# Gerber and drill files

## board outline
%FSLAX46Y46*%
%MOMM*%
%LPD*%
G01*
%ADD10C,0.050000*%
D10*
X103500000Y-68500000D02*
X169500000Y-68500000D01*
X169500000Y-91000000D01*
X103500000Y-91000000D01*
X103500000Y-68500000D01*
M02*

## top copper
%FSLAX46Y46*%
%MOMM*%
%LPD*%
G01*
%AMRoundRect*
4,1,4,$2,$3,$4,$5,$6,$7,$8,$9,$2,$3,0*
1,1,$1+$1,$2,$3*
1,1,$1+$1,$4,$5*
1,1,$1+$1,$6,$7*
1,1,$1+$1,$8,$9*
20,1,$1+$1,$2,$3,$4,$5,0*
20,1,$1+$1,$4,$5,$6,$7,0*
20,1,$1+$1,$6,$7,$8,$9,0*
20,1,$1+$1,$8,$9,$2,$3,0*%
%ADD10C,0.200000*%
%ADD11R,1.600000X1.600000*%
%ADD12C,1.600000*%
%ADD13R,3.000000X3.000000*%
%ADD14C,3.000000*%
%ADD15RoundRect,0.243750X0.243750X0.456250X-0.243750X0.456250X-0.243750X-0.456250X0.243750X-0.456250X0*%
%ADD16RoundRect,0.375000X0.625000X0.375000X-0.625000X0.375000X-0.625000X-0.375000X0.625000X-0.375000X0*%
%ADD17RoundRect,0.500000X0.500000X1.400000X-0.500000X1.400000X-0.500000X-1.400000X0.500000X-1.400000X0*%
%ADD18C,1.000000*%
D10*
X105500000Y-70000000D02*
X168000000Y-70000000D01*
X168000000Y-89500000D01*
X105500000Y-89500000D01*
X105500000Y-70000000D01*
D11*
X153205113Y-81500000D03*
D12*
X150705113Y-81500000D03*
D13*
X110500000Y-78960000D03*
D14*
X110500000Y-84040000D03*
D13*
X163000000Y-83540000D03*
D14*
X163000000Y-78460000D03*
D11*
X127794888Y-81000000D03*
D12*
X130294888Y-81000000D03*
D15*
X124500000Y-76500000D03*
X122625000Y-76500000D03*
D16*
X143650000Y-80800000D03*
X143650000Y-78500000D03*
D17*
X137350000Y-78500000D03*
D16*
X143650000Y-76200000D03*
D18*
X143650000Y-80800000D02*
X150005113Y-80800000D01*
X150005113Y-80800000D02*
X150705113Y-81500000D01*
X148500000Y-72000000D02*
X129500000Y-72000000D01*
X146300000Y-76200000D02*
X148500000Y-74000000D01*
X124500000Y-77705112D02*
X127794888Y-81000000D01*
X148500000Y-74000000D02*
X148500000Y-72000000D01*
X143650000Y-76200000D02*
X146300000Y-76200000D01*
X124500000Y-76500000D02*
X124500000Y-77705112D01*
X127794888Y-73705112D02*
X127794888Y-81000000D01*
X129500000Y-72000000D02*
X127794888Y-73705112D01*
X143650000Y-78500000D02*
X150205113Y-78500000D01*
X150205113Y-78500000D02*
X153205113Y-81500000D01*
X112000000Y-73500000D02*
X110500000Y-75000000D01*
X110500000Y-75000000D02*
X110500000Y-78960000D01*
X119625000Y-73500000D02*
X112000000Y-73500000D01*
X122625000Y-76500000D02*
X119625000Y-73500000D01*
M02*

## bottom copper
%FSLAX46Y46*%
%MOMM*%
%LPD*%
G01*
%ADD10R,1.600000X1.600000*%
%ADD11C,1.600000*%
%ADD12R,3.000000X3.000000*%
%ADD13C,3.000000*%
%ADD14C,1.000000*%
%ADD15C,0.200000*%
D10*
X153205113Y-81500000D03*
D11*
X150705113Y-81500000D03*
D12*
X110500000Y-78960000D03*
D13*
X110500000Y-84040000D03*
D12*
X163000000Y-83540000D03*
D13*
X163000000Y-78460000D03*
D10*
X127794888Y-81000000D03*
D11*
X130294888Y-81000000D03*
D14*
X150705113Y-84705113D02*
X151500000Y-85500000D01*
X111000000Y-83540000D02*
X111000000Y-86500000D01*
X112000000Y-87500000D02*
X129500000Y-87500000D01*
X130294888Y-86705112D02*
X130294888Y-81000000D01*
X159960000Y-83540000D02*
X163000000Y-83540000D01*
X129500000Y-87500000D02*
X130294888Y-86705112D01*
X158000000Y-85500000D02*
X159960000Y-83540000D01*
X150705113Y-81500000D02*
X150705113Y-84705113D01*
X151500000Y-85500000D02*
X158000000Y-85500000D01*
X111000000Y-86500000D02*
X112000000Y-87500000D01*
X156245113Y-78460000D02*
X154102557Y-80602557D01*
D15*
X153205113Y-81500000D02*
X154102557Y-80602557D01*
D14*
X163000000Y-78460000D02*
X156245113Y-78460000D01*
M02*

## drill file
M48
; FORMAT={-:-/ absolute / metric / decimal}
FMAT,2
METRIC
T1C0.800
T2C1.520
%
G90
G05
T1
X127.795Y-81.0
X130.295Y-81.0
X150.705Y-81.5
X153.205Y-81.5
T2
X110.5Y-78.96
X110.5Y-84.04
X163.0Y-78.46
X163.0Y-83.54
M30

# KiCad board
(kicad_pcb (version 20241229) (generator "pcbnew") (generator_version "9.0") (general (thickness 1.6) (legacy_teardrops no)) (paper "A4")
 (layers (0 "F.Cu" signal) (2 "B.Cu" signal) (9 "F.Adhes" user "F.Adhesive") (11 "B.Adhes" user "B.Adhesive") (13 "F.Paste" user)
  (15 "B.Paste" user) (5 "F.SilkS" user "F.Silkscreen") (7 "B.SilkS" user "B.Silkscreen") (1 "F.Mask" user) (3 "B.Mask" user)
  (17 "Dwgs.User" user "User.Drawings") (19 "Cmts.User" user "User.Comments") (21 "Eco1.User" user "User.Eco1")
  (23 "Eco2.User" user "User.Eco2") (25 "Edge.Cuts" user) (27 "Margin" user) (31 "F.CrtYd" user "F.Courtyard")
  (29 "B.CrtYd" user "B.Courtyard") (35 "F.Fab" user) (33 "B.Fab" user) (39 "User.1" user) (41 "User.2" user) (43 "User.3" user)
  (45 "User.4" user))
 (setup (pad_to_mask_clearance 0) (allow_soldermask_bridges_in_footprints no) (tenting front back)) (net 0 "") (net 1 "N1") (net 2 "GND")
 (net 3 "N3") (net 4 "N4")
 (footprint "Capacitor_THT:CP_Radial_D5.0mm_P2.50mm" (layer "F.Cu") (at 153.205113 81.5 180)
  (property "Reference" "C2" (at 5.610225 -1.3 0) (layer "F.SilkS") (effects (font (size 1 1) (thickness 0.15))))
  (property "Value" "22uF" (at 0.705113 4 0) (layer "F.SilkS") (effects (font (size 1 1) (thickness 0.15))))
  (pad "1" thru_hole rect (at 0 0 180) (size 1.6 1.6) (drill 0.8) (layers "*.Cu" "*.Mask") (remove_unused_layers no) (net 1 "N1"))
  (pad "2" thru_hole circle (at 2.5 0 180) (size 1.6 1.6) (drill 0.8) (layers "*.Cu" "*.Mask") (remove_unused_layers no) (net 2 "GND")))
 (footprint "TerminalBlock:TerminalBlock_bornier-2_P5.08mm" (layer "F.Cu") (at 110.5 78.96 -90)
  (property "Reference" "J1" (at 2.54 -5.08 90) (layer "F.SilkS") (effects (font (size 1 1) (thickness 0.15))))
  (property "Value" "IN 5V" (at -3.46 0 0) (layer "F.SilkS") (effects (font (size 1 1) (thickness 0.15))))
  (pad "1" thru_hole rect (at 0 0 270) (size 3 3) (drill 1.52) (layers "*.Cu" "*.Mask") (remove_unused_layers no) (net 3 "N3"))
  (pad "2" thru_hole circle (at 5.08 0 270) (size 3 3) (drill 1.52) (layers "*.Cu" "*.Mask") (remove_unused_layers no) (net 2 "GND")))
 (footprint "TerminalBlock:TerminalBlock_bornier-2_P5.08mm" (layer "F.Cu") (at 163 83.54 90)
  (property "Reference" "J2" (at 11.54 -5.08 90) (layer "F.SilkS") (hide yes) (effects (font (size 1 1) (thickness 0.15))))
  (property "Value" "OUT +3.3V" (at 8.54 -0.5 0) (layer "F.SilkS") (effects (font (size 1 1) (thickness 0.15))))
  (pad "1" thru_hole rect (at 0 0 90) (size 3 3) (drill 1.52) (layers "*.Cu" "*.Mask") (remove_unused_layers no) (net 2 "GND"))
  (pad "2" thru_hole circle (at 5.08 0 90) (size 3 3) (drill 1.52) (layers "*.Cu" "*.Mask") (remove_unused_layers no) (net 1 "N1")))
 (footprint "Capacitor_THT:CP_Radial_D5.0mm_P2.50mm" (layer "F.Cu") (at 127.794888 81)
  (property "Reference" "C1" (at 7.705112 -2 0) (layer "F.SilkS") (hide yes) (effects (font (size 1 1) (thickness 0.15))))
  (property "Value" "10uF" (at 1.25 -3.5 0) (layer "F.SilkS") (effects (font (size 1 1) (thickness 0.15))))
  (pad "1" thru_hole rect (at 0 0) (size 1.6 1.6) (drill 0.8) (layers "*.Cu" "*.Mask") (remove_unused_layers no) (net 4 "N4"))
  (pad "2" thru_hole circle (at 2.5 0) (size 1.6 1.6) (drill 0.8) (layers "*.Cu" "*.Mask") (remove_unused_layers no) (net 2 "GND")))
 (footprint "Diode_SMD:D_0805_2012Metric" (layer "F.Cu") (at 123.5625 76.5 180)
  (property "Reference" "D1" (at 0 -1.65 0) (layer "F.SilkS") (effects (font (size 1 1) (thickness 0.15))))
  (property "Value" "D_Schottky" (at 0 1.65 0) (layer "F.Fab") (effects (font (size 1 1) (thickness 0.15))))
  (pad "1" smd roundrect (at -0.9375 0 180) (size 0.975 1.4) (layers "F.Cu" "F.Mask" "F.Paste") (roundrect_rratio 0.25) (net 4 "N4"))
  (pad "2" smd roundrect (at 0.9375 0 180) (size 0.975 1.4) (layers "F.Cu" "F.Mask" "F.Paste") (roundrect_rratio 0.25) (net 3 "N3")))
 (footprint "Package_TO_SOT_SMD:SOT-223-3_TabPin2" (layer "F.Cu") (at 140.5 78.5 180)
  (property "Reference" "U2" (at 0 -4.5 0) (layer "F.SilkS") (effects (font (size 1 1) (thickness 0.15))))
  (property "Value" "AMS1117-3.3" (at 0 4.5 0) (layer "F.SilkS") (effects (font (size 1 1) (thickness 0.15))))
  (pad "1" smd roundrect (at -3.15 -2.3 180) (size 2 1.5) (layers "F.Cu" "F.Mask" "F.Paste") (roundrect_rratio 0.25) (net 2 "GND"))
  (pad "2" smd roundrect (at -3.15 0 180) (size 2 1.5) (layers "F.Cu" "F.Mask" "F.Paste") (roundrect_rratio 0.25) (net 1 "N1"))
  (pad "2" smd roundrect (at 3.15 0 180) (size 2 3.8) (layers "F.Cu" "F.Mask" "F.Paste") (roundrect_rratio 0.25) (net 1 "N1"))
  (pad "3" smd roundrect (at -3.15 2.3 180) (size 2 1.5) (layers "F.Cu" "F.Mask" "F.Paste") (roundrect_rratio 0.25) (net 4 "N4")))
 (gr_rect (start 105.5 70) (end 168 89.5) (stroke (width 0.2) (type default)) (fill no) (layer "F.Cu"))
 (gr_rect (start 103.5 68.5) (end 169.5 91) (stroke (width 0.05) (type default)) (fill no) (layer "Edge.Cuts"))
 (segment (start 143.65 80.8) (end 150.005113 80.8) (width 1) (layer "F.Cu") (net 2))
 (segment (start 150.005113 80.8) (end 150.705113 81.5) (width 1) (layer "F.Cu") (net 2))
 (segment (start 150.705113 84.705113) (end 151.5 85.5) (width 1) (layer "B.Cu") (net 2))
 (segment (start 111 83.54) (end 111 86.5) (width 1) (layer "B.Cu") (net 2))
 (segment (start 112 87.5) (end 129.5 87.5) (width 1) (layer "B.Cu") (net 2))
 (segment (start 130.294888 86.705112) (end 130.294888 81) (width 1) (layer "B.Cu") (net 2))
 (segment (start 159.96 83.54) (end 163 83.54) (width 1) (layer "B.Cu") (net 2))
 (segment (start 129.5 87.5) (end 130.294888 86.705112) (width 1) (layer "B.Cu") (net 2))
 (segment (start 158 85.5) (end 159.96 83.54) (width 1) (layer "B.Cu") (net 2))
 (segment (start 150.705113 81.5) (end 150.705113 84.705113) (width 1) (layer "B.Cu") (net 2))
 (segment (start 151.5 85.5) (end 158 85.5) (width 1) (layer "B.Cu") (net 2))
 (segment (start 111 86.5) (end 112 87.5) (width 1) (layer "B.Cu") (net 2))
 (segment (start 148.5 72) (end 129.5 72) (width 1) (layer "F.Cu") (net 4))
 (segment (start 146.3 76.2) (end 148.5 74) (width 1) (layer "F.Cu") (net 4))
 (segment (start 124.5 77.705112) (end 127.794888 81) (width 1) (layer "F.Cu") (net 4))
 (segment (start 148.5 74) (end 148.5 72) (width 1) (layer "F.Cu") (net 4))
 (segment (start 143.65 76.2) (end 146.3 76.2) (width 1) (layer "F.Cu") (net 4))
 (segment (start 124.5 76.5) (end 124.5 77.705112) (width 1) (layer "F.Cu") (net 4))
 (segment (start 127.794888 73.705112) (end 127.794888 81) (width 1) (layer "F.Cu") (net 4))
 (segment (start 129.5 72) (end 127.794888 73.705112) (width 1) (layer "F.Cu") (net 4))
 (segment (start 143.65 78.5) (end 150.205113 78.5) (width 1) (layer "F.Cu") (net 1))
 (segment (start 150.205113 78.5) (end 153.205113 81.5) (width 1) (layer "F.Cu") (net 1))
 (segment (start 156.245113 78.46) (end 154.102557 80.602557) (width 1) (layer "B.Cu") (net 1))
 (segment (start 153.205113 81.5) (end 154.102557 80.602557) (width 0.2) (layer "B.Cu") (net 1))
 (segment (start 163 78.46) (end 156.245113 78.46) (width 1) (layer "B.Cu") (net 1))
 (segment (start 112 73.5) (end 110.5 75) (width 1) (layer "F.Cu") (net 3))
 (segment (start 110.5 75) (end 110.5 78.96) (width 1) (layer "F.Cu") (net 3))
 (segment (start 119.625 73.5) (end 112 73.5) (width 1) (layer "F.Cu") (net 3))
 (segment (start 122.625 76.5) (end 119.625 73.5) (width 1) (layer "F.Cu") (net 3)))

